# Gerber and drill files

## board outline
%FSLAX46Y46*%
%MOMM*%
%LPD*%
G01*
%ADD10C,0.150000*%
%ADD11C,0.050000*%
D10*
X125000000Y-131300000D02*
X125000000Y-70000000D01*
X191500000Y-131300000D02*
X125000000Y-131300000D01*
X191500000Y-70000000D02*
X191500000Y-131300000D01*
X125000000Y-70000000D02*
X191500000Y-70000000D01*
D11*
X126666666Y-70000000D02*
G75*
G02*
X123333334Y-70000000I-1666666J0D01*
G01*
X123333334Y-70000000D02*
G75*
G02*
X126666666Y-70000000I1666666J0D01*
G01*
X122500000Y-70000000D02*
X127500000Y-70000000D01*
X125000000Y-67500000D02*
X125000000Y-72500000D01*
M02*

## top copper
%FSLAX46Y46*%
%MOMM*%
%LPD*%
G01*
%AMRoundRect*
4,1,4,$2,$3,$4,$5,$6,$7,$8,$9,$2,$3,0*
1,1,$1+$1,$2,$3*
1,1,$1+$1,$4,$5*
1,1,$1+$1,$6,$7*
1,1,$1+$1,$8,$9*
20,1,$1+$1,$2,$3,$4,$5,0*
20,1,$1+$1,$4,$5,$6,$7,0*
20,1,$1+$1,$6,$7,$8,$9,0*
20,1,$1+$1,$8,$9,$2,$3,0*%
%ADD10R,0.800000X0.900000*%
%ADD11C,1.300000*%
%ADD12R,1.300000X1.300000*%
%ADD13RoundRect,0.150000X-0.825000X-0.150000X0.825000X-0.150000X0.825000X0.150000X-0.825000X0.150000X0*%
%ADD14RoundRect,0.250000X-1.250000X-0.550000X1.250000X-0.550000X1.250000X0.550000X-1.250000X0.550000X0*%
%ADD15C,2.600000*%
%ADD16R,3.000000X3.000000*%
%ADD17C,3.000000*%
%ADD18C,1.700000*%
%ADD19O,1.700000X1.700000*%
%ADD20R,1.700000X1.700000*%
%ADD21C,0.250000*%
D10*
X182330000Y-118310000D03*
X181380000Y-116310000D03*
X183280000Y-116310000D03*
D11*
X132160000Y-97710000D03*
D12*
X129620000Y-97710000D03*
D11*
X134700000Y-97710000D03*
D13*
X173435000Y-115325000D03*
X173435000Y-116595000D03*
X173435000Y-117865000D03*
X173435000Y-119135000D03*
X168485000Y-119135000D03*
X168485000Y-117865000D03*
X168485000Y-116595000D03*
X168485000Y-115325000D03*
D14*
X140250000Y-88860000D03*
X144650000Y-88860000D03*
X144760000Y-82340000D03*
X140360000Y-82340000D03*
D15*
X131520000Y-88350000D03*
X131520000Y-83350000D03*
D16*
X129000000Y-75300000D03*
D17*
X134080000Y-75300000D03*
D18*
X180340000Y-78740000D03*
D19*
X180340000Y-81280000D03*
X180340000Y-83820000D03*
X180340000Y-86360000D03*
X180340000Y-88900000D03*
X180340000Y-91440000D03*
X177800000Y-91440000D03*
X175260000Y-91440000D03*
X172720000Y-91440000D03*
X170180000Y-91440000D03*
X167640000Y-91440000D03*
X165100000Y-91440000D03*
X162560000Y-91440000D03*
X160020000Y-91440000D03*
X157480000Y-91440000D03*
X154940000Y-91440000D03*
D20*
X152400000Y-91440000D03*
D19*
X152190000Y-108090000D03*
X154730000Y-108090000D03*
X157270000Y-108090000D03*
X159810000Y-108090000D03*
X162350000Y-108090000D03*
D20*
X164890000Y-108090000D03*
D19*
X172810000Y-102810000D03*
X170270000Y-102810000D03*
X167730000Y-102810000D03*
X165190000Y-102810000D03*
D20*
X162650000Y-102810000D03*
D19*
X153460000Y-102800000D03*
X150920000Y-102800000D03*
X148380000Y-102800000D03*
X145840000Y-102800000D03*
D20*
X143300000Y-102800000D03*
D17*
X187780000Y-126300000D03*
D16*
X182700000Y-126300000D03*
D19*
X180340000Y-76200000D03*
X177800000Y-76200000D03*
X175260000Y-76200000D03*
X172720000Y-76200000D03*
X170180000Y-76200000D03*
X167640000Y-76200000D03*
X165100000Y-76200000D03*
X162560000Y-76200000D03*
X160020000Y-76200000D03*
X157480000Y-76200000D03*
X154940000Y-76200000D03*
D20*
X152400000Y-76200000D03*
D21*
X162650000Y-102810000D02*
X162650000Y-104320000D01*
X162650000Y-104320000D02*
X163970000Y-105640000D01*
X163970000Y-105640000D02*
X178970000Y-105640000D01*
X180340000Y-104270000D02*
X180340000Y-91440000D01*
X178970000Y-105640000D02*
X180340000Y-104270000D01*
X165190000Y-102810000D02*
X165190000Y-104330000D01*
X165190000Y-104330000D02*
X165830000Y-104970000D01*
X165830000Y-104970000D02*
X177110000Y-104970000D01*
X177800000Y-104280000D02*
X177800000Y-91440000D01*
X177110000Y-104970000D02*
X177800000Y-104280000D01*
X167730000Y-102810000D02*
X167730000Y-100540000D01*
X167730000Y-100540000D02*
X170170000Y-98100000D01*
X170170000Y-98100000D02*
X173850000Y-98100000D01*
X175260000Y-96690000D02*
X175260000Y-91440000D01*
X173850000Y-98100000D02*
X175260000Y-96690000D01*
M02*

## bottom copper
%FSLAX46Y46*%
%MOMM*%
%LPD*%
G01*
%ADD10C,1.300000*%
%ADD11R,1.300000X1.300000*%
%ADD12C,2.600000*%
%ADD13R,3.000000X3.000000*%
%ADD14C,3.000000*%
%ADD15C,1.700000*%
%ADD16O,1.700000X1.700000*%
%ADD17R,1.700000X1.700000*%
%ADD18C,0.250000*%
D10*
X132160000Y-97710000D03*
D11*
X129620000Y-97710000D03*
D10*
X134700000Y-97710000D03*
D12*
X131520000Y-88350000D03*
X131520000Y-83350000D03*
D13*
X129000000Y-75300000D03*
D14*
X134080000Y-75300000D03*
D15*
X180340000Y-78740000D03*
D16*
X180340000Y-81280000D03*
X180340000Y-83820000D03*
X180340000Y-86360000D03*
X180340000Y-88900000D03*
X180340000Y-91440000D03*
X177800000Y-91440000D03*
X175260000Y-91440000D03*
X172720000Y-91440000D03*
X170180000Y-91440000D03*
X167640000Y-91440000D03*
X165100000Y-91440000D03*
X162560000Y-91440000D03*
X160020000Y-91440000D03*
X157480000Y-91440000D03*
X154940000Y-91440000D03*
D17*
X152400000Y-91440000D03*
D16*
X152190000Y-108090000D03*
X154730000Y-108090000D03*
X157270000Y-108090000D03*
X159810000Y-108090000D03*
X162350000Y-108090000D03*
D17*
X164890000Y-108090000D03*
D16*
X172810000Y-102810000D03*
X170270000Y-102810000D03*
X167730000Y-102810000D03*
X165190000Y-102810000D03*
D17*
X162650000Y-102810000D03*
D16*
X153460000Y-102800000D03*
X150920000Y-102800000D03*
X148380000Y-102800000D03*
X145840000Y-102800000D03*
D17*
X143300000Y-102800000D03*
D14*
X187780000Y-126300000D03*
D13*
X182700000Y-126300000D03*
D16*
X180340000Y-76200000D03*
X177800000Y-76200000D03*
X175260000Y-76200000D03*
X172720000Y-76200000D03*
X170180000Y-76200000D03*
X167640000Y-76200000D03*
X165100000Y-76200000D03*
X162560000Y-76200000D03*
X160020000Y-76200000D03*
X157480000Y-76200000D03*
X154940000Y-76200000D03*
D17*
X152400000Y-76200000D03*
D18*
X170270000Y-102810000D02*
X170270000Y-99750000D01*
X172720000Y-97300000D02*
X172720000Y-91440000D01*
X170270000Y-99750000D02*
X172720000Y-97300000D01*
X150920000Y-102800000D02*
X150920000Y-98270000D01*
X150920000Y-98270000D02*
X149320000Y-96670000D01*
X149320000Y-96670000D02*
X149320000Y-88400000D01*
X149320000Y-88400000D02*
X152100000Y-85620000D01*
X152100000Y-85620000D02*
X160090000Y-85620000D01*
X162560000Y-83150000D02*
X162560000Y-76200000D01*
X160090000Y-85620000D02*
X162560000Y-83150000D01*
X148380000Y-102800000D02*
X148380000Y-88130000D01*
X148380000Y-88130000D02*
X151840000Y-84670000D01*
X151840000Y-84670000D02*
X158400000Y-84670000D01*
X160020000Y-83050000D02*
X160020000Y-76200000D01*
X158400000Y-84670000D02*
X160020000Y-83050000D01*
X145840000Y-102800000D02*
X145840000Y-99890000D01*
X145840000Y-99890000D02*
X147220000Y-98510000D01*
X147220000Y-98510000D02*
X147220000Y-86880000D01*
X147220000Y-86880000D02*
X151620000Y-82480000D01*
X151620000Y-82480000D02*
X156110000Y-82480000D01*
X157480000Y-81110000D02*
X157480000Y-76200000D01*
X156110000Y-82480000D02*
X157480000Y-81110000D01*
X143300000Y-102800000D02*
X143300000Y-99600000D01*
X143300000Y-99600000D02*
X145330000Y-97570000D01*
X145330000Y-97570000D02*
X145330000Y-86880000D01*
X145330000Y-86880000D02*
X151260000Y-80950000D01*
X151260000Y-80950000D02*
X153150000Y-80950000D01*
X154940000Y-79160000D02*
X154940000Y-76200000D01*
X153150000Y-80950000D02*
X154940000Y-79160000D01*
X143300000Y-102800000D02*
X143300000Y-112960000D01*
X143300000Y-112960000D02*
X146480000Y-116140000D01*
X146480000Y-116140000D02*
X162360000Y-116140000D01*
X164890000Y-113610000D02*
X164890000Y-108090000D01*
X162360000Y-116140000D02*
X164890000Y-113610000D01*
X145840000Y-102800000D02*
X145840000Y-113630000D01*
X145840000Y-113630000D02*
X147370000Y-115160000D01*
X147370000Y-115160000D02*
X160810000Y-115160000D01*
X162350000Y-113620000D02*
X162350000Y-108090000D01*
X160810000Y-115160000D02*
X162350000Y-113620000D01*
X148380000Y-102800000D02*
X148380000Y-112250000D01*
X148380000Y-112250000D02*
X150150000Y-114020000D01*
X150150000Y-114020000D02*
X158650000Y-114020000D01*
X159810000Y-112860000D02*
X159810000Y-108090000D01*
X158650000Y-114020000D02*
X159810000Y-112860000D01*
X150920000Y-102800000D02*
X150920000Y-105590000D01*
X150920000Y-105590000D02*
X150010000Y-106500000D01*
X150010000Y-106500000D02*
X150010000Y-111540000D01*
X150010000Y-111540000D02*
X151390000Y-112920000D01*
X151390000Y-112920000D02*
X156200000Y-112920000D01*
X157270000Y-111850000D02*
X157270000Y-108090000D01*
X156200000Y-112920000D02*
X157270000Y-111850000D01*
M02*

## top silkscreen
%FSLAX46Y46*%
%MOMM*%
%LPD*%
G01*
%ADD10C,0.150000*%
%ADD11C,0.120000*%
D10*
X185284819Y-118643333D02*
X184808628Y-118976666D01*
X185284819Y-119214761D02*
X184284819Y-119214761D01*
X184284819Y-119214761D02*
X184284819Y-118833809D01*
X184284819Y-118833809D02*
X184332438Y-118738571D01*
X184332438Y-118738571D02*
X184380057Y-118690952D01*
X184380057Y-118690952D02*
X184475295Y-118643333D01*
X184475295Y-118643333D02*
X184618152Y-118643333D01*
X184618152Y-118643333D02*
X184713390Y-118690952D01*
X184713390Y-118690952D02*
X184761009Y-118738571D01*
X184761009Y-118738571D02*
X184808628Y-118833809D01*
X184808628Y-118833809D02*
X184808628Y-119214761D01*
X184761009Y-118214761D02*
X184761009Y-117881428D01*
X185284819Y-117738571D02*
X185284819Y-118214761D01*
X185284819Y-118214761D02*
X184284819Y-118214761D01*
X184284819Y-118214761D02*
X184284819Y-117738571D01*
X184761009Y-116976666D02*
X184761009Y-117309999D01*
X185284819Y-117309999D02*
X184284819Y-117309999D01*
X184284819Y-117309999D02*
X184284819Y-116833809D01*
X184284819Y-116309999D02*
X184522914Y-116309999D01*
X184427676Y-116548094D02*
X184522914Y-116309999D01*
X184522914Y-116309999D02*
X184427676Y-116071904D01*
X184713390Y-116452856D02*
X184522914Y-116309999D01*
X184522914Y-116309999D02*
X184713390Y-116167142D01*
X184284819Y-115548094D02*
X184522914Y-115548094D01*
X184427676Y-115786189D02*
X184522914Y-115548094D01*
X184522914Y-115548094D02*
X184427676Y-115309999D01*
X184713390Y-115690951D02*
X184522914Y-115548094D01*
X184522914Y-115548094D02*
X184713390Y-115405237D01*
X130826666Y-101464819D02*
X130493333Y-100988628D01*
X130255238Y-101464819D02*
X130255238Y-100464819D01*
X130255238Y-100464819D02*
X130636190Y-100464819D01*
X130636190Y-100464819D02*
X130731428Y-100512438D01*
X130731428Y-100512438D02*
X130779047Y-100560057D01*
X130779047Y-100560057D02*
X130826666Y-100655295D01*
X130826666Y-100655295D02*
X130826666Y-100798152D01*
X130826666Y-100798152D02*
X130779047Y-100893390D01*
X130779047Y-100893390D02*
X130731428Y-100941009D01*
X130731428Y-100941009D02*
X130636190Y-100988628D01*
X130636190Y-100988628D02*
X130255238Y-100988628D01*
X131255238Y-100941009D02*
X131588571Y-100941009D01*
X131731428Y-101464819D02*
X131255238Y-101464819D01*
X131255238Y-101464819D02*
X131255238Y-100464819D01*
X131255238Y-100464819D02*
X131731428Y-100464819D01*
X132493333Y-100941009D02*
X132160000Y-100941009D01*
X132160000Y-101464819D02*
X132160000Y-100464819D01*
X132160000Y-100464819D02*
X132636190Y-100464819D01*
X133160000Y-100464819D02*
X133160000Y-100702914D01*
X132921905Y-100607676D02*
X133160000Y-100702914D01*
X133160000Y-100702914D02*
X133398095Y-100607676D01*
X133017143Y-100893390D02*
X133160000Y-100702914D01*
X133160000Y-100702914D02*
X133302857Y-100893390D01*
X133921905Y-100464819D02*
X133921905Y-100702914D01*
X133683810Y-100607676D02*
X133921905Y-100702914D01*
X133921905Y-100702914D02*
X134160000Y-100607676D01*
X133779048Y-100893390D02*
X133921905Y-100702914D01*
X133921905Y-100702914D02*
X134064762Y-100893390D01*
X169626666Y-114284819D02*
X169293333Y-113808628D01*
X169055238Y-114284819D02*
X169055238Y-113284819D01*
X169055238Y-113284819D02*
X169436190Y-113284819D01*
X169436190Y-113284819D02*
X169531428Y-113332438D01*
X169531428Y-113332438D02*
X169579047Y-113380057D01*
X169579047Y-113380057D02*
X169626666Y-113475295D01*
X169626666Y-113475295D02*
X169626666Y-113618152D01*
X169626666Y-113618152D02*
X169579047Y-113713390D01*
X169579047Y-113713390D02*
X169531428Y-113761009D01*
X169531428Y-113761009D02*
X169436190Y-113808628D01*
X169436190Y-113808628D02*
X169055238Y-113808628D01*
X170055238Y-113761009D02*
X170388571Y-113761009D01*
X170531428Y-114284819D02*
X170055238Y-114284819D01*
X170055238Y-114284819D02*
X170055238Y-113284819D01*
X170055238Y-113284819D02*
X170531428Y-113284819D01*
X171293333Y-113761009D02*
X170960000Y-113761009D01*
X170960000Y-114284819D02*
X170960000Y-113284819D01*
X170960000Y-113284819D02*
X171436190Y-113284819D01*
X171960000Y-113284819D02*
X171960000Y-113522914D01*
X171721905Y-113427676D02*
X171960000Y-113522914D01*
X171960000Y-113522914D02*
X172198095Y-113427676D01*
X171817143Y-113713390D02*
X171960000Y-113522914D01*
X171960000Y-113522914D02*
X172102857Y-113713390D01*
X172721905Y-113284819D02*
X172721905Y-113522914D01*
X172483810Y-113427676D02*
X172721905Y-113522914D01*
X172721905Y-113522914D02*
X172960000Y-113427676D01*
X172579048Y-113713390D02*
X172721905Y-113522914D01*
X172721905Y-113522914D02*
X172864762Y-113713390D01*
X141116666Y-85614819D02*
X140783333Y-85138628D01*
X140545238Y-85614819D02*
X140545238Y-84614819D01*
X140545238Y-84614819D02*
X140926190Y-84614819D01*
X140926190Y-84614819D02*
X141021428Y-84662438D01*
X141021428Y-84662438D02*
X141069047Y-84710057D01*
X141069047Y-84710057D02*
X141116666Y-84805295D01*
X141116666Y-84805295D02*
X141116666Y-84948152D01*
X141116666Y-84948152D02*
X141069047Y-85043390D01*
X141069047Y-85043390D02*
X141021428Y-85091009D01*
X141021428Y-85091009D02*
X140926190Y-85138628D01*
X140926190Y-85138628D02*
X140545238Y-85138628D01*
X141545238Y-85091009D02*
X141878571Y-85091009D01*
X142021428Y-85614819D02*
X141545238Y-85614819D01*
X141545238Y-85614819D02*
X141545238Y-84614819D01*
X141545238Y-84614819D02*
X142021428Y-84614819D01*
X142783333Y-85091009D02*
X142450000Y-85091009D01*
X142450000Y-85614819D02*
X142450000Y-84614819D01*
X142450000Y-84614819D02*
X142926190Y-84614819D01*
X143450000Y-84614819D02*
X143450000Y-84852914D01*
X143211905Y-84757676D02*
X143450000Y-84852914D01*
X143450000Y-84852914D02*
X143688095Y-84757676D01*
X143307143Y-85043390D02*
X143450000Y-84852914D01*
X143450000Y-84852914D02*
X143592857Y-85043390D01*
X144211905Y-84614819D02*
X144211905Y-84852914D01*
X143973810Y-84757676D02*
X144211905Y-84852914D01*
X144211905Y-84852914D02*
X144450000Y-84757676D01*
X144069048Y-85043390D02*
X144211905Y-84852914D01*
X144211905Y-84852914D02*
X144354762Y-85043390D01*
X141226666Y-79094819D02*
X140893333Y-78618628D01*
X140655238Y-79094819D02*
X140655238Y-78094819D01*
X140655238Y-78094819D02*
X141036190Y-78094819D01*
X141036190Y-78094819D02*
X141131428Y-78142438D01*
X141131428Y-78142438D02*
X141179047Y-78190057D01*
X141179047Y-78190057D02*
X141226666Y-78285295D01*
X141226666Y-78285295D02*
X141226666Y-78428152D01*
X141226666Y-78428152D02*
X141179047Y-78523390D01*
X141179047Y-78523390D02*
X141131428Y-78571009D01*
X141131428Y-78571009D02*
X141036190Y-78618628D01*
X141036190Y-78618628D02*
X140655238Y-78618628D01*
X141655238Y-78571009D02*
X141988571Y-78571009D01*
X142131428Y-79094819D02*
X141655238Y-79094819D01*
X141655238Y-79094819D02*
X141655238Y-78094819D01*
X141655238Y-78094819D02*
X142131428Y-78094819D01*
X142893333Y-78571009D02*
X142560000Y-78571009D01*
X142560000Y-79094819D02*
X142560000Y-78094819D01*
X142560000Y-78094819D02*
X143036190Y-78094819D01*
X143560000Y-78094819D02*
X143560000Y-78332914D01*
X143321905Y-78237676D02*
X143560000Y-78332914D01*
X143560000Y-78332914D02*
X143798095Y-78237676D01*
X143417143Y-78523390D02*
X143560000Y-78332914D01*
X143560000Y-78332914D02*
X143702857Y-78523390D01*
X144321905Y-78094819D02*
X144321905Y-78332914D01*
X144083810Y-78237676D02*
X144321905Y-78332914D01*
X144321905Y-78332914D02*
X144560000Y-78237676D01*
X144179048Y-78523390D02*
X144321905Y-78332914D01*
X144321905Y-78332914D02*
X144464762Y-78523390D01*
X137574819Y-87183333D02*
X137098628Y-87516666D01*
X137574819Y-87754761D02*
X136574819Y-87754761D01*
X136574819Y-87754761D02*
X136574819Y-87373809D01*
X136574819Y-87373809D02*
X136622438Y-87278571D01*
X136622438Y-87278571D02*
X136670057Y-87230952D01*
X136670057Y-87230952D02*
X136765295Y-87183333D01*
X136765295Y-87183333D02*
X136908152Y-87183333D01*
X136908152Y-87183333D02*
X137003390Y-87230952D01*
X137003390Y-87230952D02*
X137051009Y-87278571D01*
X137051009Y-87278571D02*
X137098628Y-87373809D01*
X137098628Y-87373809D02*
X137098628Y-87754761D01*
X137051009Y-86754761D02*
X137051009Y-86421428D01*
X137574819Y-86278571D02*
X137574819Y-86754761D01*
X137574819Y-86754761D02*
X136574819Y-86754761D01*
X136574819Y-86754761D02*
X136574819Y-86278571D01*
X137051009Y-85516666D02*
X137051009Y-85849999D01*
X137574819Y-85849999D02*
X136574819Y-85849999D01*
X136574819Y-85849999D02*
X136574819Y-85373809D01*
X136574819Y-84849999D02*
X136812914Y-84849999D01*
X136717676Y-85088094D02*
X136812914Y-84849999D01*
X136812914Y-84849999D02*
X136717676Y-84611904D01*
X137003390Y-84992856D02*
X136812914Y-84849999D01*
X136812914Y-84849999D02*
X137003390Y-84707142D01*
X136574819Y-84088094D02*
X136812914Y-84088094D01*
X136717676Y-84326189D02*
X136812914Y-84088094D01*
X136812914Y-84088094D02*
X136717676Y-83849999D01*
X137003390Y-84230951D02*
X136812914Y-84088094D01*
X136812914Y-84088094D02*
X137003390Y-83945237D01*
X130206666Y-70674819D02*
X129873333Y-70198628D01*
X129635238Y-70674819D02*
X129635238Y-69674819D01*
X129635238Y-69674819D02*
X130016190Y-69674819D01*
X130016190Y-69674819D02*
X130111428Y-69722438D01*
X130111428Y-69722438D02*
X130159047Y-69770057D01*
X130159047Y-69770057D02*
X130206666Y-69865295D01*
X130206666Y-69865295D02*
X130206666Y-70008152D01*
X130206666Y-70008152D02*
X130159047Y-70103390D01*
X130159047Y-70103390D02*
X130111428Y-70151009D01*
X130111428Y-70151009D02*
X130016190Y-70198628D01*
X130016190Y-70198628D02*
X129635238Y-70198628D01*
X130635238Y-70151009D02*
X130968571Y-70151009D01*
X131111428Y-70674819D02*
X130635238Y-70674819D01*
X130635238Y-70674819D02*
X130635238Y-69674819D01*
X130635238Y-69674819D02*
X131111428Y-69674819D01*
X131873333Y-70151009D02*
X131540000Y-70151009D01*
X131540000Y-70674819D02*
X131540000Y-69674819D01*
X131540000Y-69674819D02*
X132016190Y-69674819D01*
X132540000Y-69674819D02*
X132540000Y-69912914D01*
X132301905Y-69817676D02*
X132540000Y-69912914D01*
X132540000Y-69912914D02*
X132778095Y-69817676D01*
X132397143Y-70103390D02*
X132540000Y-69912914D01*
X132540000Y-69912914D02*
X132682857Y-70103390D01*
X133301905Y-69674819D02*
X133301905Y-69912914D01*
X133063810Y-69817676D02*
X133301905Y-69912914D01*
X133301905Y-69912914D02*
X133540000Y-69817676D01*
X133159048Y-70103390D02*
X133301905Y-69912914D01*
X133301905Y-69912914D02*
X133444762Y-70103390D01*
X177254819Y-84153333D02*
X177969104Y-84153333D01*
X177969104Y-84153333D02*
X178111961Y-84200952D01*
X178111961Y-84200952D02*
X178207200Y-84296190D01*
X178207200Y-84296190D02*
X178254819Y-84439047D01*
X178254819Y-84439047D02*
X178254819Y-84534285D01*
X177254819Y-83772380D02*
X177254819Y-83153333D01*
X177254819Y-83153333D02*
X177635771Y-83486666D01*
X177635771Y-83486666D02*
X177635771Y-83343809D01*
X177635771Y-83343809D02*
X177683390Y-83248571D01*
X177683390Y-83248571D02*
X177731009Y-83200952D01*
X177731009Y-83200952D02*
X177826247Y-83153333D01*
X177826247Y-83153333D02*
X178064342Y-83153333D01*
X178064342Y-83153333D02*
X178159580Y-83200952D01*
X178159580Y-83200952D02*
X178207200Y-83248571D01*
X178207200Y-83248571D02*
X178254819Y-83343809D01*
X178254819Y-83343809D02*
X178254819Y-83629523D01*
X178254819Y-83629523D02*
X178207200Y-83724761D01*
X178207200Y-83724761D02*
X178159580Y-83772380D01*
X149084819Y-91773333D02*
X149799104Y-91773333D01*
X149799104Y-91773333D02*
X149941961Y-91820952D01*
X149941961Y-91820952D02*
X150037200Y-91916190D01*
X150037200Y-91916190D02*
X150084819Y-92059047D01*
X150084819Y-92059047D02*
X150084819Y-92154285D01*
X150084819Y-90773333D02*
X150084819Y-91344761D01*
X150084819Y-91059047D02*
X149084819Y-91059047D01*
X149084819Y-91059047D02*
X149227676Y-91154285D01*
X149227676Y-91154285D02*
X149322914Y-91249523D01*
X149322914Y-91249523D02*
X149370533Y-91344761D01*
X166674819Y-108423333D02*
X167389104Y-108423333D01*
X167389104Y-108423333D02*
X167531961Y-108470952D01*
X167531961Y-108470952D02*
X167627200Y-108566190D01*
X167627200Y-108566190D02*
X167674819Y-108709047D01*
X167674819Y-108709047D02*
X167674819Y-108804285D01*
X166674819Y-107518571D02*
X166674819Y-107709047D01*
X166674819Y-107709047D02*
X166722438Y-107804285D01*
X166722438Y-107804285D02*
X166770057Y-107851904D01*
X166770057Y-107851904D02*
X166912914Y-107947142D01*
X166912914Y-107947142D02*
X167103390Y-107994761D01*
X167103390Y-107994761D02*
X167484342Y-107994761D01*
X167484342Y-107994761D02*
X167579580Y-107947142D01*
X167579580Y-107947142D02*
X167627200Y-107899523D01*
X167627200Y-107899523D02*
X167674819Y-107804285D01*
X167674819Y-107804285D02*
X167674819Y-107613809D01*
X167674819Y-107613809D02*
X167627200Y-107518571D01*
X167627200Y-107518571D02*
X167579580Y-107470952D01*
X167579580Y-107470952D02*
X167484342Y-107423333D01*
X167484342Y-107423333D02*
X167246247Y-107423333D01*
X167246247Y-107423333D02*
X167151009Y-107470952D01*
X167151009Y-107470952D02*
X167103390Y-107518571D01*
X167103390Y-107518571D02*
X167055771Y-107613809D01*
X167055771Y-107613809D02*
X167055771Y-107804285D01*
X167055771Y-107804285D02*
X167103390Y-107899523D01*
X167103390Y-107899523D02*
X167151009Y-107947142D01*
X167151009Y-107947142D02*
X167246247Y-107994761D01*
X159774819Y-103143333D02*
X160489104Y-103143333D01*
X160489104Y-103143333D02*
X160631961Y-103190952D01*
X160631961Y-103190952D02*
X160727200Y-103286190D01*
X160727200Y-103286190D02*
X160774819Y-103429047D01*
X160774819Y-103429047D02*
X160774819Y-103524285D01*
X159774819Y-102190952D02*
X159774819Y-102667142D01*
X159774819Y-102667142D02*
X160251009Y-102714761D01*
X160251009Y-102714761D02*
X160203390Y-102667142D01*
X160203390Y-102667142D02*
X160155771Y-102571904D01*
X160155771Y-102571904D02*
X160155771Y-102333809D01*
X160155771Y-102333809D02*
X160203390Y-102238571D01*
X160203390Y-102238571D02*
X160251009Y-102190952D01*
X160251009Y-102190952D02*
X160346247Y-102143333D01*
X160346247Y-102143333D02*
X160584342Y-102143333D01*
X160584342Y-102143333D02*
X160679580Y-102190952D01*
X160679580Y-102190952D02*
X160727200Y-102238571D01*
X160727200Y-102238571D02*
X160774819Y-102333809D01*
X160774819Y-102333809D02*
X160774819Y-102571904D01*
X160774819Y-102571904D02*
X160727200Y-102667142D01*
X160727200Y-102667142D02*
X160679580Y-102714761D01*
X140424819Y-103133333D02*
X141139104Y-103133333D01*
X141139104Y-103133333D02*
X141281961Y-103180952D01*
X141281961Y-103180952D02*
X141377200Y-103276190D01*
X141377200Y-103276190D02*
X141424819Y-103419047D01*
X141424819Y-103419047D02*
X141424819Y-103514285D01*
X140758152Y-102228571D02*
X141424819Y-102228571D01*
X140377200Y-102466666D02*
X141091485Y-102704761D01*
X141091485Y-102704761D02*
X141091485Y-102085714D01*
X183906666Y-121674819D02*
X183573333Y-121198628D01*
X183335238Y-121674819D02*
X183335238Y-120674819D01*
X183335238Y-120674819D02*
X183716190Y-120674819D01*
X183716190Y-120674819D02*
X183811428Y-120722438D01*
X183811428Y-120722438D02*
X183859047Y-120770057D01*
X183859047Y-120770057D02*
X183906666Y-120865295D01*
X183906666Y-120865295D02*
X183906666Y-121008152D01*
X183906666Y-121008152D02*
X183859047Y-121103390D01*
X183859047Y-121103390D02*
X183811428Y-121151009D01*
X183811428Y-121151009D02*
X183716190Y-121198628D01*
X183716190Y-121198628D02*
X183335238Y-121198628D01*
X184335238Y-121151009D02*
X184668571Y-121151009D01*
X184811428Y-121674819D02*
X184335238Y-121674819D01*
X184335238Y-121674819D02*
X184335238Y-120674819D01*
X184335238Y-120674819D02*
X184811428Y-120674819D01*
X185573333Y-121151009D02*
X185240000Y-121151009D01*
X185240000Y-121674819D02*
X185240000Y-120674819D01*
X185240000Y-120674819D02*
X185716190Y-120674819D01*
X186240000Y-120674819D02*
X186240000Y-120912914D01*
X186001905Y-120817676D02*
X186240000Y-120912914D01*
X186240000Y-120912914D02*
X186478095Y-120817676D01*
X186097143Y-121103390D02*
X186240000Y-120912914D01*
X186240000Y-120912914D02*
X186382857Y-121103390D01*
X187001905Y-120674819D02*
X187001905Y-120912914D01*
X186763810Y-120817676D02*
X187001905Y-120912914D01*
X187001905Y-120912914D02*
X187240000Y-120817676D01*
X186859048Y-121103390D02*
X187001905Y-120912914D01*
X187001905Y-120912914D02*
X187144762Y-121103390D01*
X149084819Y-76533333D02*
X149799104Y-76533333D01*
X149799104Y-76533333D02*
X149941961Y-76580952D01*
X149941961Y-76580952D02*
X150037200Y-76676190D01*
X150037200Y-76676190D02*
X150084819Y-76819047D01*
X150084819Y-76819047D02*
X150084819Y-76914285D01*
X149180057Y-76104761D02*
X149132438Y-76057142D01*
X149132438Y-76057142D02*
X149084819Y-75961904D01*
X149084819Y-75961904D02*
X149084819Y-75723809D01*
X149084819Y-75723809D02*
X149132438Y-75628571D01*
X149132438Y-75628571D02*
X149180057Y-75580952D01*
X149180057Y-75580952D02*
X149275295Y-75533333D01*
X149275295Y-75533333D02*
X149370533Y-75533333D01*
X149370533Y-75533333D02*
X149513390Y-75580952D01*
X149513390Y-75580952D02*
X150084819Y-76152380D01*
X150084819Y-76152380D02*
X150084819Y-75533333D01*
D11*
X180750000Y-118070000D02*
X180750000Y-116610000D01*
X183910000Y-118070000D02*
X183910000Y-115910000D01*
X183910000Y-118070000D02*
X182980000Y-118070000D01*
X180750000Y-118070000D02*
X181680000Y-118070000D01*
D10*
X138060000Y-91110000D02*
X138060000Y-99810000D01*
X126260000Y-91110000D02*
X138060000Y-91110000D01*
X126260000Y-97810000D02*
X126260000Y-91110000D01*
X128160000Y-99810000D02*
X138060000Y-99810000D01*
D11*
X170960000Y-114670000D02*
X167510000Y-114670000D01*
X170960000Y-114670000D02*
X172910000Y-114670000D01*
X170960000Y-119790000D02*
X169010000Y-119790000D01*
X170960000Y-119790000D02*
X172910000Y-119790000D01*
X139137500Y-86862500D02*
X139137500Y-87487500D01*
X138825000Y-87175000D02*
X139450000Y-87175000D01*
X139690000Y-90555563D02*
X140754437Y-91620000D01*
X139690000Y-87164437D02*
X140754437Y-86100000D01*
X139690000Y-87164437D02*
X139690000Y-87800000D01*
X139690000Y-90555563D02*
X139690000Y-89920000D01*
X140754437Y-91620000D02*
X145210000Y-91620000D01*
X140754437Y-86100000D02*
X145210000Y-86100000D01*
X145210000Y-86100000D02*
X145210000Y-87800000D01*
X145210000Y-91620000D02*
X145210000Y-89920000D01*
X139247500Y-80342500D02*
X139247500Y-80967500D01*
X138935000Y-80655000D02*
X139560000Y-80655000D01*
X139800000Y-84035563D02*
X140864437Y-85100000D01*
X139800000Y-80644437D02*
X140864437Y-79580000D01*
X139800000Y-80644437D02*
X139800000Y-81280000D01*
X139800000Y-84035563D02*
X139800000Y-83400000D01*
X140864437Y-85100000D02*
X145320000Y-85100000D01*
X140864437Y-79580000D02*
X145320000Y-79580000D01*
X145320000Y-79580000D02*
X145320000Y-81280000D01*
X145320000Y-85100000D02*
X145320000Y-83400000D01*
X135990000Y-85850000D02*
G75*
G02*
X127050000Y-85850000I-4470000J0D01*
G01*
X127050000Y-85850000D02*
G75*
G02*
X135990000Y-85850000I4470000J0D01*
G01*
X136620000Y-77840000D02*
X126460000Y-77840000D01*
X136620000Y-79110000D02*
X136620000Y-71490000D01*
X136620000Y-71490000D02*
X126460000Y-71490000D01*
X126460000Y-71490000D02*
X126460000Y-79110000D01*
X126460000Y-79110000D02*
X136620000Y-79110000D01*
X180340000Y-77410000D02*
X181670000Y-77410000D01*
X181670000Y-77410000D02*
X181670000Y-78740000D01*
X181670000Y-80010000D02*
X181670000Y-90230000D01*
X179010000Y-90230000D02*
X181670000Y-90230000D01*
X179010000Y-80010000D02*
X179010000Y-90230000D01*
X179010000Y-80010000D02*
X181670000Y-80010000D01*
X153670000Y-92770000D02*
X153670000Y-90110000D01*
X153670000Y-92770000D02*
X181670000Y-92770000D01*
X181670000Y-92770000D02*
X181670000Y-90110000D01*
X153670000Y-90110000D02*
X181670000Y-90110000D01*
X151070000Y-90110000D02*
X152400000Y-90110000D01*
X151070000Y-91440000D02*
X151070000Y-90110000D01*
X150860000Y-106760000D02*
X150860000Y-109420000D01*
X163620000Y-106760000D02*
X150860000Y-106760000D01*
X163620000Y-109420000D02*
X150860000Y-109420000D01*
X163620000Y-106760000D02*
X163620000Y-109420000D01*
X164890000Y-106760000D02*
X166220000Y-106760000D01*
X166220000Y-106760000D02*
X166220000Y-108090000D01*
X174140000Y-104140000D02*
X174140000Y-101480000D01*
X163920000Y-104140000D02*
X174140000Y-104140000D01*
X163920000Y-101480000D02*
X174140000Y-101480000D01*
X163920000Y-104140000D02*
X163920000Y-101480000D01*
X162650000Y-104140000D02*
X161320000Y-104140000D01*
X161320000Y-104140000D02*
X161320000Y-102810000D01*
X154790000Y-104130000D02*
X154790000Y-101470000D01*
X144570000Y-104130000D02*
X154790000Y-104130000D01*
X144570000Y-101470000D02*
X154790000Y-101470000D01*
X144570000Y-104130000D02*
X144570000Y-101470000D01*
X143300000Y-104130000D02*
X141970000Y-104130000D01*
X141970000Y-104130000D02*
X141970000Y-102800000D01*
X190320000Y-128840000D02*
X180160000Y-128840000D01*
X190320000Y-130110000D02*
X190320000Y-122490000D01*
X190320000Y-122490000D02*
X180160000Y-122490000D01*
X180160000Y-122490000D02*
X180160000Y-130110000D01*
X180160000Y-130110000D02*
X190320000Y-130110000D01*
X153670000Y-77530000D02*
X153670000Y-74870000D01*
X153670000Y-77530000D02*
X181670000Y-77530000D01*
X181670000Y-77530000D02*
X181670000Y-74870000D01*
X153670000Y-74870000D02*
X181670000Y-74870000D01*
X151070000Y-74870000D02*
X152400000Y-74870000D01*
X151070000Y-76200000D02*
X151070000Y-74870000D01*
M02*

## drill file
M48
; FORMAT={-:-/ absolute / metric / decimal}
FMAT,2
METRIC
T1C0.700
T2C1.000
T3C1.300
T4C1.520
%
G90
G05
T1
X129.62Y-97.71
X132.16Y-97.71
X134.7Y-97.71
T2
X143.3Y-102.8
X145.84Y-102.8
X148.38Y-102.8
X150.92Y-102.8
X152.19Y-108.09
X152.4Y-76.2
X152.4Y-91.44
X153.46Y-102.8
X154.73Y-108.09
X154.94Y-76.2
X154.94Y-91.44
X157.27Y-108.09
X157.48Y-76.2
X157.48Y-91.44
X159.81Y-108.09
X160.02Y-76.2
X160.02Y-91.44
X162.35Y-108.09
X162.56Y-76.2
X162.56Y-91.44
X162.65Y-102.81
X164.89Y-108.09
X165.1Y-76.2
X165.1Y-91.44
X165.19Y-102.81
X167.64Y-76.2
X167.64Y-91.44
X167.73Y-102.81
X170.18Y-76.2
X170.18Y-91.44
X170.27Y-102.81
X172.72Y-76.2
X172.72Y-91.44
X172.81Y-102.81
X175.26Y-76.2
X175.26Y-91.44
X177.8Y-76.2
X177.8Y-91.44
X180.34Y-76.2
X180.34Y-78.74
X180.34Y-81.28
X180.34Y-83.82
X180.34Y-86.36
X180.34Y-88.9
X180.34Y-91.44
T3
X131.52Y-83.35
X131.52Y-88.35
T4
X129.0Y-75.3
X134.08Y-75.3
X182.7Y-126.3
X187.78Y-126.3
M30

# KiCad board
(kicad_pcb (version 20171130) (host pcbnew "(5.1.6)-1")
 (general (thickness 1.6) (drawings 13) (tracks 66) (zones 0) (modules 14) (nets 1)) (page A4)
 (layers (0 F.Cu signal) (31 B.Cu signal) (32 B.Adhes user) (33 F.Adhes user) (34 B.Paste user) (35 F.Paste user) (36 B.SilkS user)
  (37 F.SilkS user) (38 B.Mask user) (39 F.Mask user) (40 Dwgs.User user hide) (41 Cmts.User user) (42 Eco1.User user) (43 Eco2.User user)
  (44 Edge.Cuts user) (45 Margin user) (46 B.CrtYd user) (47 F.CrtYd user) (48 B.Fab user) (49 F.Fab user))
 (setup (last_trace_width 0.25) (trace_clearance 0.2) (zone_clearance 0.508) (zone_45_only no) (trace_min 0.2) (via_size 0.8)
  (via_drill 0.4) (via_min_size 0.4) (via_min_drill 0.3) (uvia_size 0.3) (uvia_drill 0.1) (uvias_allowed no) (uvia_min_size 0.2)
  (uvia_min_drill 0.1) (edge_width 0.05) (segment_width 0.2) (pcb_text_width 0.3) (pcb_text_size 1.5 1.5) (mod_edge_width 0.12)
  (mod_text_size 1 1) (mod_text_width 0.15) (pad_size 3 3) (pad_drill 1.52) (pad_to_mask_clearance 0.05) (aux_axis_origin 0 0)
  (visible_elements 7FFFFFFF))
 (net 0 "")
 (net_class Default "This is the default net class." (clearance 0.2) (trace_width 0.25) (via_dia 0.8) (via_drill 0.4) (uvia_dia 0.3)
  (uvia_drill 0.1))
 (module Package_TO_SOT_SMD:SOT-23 (layer F.Cu) (at 182.33 117.31 270)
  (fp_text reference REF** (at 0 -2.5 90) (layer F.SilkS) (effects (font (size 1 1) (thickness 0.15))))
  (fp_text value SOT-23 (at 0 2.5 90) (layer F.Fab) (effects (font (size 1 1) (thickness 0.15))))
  (fp_line (start 0.76 1.58) (end -0.7 1.58) (layer F.SilkS) (width 0.12))
  (fp_line (start 0.76 -1.58) (end -1.4 -1.58) (layer F.SilkS) (width 0.12))
  (fp_line (start 0.76 -1.58) (end 0.76 -0.65) (layer F.SilkS) (width 0.12))
  (fp_line (start 0.76 1.58) (end 0.76 0.65) (layer F.SilkS) (width 0.12))
  (pad 3 smd rect (at 1 0 270) (size 0.9 0.8) (layers F.Cu F.Paste F.Mask))
  (pad 2 smd rect (at -1 0.95 270) (size 0.9 0.8) (layers F.Cu F.Paste F.Mask))
  (pad 1 smd rect (at -1 -0.95 270) (size 0.9 0.8) (layers F.Cu F.Paste F.Mask)))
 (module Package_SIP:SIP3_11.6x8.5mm (layer F.Cu) (at 129.62 97.71)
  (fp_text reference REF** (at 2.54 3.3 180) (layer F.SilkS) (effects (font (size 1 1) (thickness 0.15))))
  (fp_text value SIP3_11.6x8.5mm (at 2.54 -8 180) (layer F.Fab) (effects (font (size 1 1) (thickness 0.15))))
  (fp_line (start 8.44 -6.6) (end 8.44 2.1) (layer F.SilkS) (width 0.15))
  (fp_line (start -3.36 -6.6) (end 8.44 -6.6) (layer F.SilkS) (width 0.15))
  (fp_line (start -3.36 0.1) (end -3.36 -6.6) (layer F.SilkS) (width 0.15))
  (fp_line (start -1.46 2.1) (end 8.44 2.1) (layer F.SilkS) (width 0.15))
  (pad 2 thru_hole circle (at 2.54 0 180) (size 1.3 1.3) (drill 0.7) (layers *.Cu *.Mask))
  (pad 1 thru_hole rect (at 0 0 270) (size 1.3 1.3) (drill 0.7) (layers *.Cu *.Mask))
  (pad 3 thru_hole circle (at 5.08 0 270) (size 1.3 1.3) (drill 0.7) (layers *.Cu *.Mask)))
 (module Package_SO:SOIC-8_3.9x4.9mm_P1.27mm (layer F.Cu) (at 170.96 117.23)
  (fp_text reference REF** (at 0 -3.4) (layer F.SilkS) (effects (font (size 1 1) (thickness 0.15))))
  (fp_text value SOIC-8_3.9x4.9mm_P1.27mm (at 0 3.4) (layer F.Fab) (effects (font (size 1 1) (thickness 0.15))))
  (fp_line (start 0 -2.56) (end -3.45 -2.56) (layer F.SilkS) (width 0.12))
  (fp_line (start 0 -2.56) (end 1.95 -2.56) (layer F.SilkS) (width 0.12))
  (fp_line (start 0 2.56) (end -1.95 2.56) (layer F.SilkS) (width 0.12))
  (fp_line (start 0 2.56) (end 1.95 2.56) (layer F.SilkS) (width 0.12))
  (pad 8 smd roundrect (at 2.475 -1.905) (size 1.95 0.6) (layers F.Cu F.Paste F.Mask) (roundrect_rratio 0.25))
  (pad 7 smd roundrect (at 2.475 -0.635) (size 1.95 0.6) (layers F.Cu F.Paste F.Mask) (roundrect_rratio 0.25))
  (pad 6 smd roundrect (at 2.475 0.635) (size 1.95 0.6) (layers F.Cu F.Paste F.Mask) (roundrect_rratio 0.25))
  (pad 5 smd roundrect (at 2.475 1.905) (size 1.95 0.6) (layers F.Cu F.Paste F.Mask) (roundrect_rratio 0.25))
  (pad 4 smd roundrect (at -2.475 1.905) (size 1.95 0.6) (layers F.Cu F.Paste F.Mask) (roundrect_rratio 0.25))
  (pad 3 smd roundrect (at -2.475 0.635) (size 1.95 0.6) (layers F.Cu F.Paste F.Mask) (roundrect_rratio 0.25))
  (pad 2 smd roundrect (at -2.475 -0.635) (size 1.95 0.6) (layers F.Cu F.Paste F.Mask) (roundrect_rratio 0.25))
  (pad 1 smd roundrect (at -2.475 -1.905) (size 1.95 0.6) (layers F.Cu F.Paste F.Mask) (roundrect_rratio 0.25)))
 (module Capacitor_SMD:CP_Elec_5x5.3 (layer F.Cu) (at 142.45 88.86)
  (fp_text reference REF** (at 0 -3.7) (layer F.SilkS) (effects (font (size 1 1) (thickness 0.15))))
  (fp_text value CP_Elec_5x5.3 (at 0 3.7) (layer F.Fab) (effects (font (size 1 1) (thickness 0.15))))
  (fp_line (start -3.3125 -1.9975) (end -3.3125 -1.3725) (layer F.SilkS) (width 0.12))
  (fp_line (start -3.625 -1.685) (end -3 -1.685) (layer F.SilkS) (width 0.12))
  (fp_line (start -2.76 1.695563) (end -1.695563 2.76) (layer F.SilkS) (width 0.12))
  (fp_line (start -2.76 -1.695563) (end -1.695563 -2.76) (layer F.SilkS) (width 0.12))
  (fp_line (start -2.76 -1.695563) (end -2.76 -1.06) (layer F.SilkS) (width 0.12))
  (fp_line (start -2.76 1.695563) (end -2.76 1.06) (layer F.SilkS) (width 0.12))
  (fp_line (start -1.695563 2.76) (end 2.76 2.76) (layer F.SilkS) (width 0.12))
  (fp_line (start -1.695563 -2.76) (end 2.76 -2.76) (layer F.SilkS) (width 0.12))
  (fp_line (start 2.76 -2.76) (end 2.76 -1.06) (layer F.SilkS) (width 0.12))
  (fp_line (start 2.76 2.76) (end 2.76 1.06) (layer F.SilkS) (width 0.12))
  (pad 1 smd roundrect (at -2.2 0) (size 3 1.6) (layers F.Cu F.Paste F.Mask) (roundrect_rratio 0.15625))
  (pad 2 smd roundrect (at 2.2 0) (size 3 1.6) (layers F.Cu F.Paste F.Mask) (roundrect_rratio 0.15625)))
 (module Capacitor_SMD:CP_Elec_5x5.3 (layer F.Cu) (at 142.56 82.34)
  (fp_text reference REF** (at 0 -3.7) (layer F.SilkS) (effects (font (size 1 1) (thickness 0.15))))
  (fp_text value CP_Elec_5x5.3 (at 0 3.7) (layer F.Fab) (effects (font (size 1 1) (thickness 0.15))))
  (fp_line (start -3.3125 -1.9975) (end -3.3125 -1.3725) (layer F.SilkS) (width 0.12))
  (fp_line (start -3.625 -1.685) (end -3 -1.685) (layer F.SilkS) (width 0.12))
  (fp_line (start -2.76 1.695563) (end -1.695563 2.76) (layer F.SilkS) (width 0.12))
  (fp_line (start -2.76 -1.695563) (end -1.695563 -2.76) (layer F.SilkS) (width 0.12))
  (fp_line (start -2.76 -1.695563) (end -2.76 -1.06) (layer F.SilkS) (width 0.12))
  (fp_line (start -2.76 1.695563) (end -2.76 1.06) (layer F.SilkS) (width 0.12))
  (fp_line (start -1.695563 2.76) (end 2.76 2.76) (layer F.SilkS) (width 0.12))
  (fp_line (start -1.695563 -2.76) (end 2.76 -2.76) (layer F.SilkS) (width 0.12))
  (fp_line (start 2.76 -2.76) (end 2.76 -1.06) (layer F.SilkS) (width 0.12))
  (fp_line (start 2.76 2.76) (end 2.76 1.06) (layer F.SilkS) (width 0.12))
  (pad 2 smd roundrect (at 2.2 0) (size 3 1.6) (layers F.Cu F.Paste F.Mask) (roundrect_rratio 0.15625))
  (pad 1 smd roundrect (at -2.2 0) (size 3 1.6) (layers F.Cu F.Paste F.Mask) (roundrect_rratio 0.15625)))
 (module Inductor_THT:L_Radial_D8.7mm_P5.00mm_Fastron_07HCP (layer F.Cu) (at 131.52 83.35 270)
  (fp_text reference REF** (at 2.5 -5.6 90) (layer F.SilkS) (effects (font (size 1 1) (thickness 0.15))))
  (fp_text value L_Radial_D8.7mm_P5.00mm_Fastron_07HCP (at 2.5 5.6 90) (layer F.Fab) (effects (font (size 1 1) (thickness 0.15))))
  (fp_circle (center 2.5 0) (end 6.97 0) (layer F.SilkS) (width 0.12))
  (pad 2 thru_hole circle (at 5 0 270) (size 2.6 2.6) (drill 1.3) (layers *.Cu *.Mask))
  (pad 1 thru_hole circle (at 0 0 270) (size 2.6 2.6) (drill 1.3) (layers *.Cu *.Mask)))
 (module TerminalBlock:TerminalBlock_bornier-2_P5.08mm (layer F.Cu) (at 129 75.3)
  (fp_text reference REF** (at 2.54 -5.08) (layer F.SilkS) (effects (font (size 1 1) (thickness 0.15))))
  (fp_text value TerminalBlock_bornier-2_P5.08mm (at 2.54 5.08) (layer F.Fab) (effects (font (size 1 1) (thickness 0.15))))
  (fp_line (start 7.62 2.54) (end -2.54 2.54) (layer F.SilkS) (width 0.12))
  (fp_line (start 7.62 3.81) (end 7.62 -3.81) (layer F.SilkS) (width 0.12))
  (fp_line (start 7.62 -3.81) (end -2.54 -3.81) (layer F.SilkS) (width 0.12))
  (fp_line (start -2.54 -3.81) (end -2.54 3.81) (layer F.SilkS) (width 0.12))
  (fp_line (start -2.54 3.81) (end 7.62 3.81) (layer F.SilkS) (width 0.12))
  (pad VCC thru_hole rect (at 0 0) (size 3 3) (drill 1.52) (layers *.Cu *.Mask))
  (pad GND thru_hole circle (at 5.08 0) (size 3 3) (drill 1.52) (layers *.Cu *.Mask)))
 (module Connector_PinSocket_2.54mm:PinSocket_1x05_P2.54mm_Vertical (layer F.Cu) (at 180.34 78.74)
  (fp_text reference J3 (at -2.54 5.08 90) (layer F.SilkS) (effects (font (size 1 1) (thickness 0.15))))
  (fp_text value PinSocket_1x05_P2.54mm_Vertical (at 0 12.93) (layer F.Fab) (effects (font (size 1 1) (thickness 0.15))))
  (fp_line (start 0 -1.33) (end 1.33 -1.33) (layer F.SilkS) (width 0.12))
  (fp_line (start 1.33 -1.33) (end 1.33 0) (layer F.SilkS) (width 0.12))
  (fp_line (start 1.33 1.27) (end 1.33 11.49) (layer F.SilkS) (width 0.12))
  (fp_line (start -1.33 11.49) (end 1.33 11.49) (layer F.SilkS) (width 0.12))
  (fp_line (start -1.33 1.27) (end -1.33 11.49) (layer F.SilkS) (width 0.12))
  (fp_line (start -1.33 1.27) (end 1.33 1.27) (layer F.SilkS) (width 0.12))
  (pad TDO thru_hole circle (at 0 0) (size 1.7 1.7) (drill 1) (layers *.Cu *.Mask))
  (pad GND thru_hole oval (at 0 2.54) (size 1.7 1.7) (drill 1) (layers *.Cu *.Mask))
  (pad TDI thru_hole oval (at 0 5.08) (size 1.7 1.7) (drill 1) (layers *.Cu *.Mask))
  (pad TCK thru_hole oval (at 0 7.62) (size 1.7 1.7) (drill 1) (layers *.Cu *.Mask))
  (pad TMS thru_hole oval (at 0 10.16) (size 1.7 1.7) (drill 1) (layers *.Cu *.Mask)))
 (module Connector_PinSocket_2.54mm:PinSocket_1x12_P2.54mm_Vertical (layer F.Cu) (at 152.4 91.44 90)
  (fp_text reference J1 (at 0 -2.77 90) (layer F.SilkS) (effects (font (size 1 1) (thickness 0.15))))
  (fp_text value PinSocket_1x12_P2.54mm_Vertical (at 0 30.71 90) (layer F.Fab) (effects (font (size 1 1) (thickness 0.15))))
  (fp_line (start -1.33 1.27) (end 1.33 1.27) (layer F.SilkS) (width 0.12))
  (fp_line (start -1.33 1.27) (end -1.33 29.27) (layer F.SilkS) (width 0.12))
  (fp_line (start -1.33 29.27) (end 1.33 29.27) (layer F.SilkS) (width 0.12))
  (fp_line (start 1.33 1.27) (end 1.33 29.27) (layer F.SilkS) (width 0.12))
  (fp_line (start 1.33 -1.33) (end 1.33 0) (layer F.SilkS) (width 0.12))
  (fp_line (start 0 -1.33) (end 1.33 -1.33) (layer F.SilkS) (width 0.12))
  (pad taster0 thru_hole oval (at 0 27.94 90) (size 1.7 1.7) (drill 1) (layers *.Cu *.Mask))
  (pad taster1 thru_hole oval (at 0 25.4 90) (size 1.7 1.7) (drill 1) (layers *.Cu *.Mask))
  (pad taster2 thru_hole oval (at 0 22.86 90) (size 1.7 1.7) (drill 1) (layers *.Cu *.Mask))
  (pad taster3 thru_hole oval (at 0 20.32 90) (size 1.7 1.7) (drill 1) (layers *.Cu *.Mask))
  (pad 8 thru_hole oval (at 0 17.78 90) (size 1.7 1.7) (drill 1) (layers *.Cu *.Mask))
  (pad 7 thru_hole oval (at 0 15.24 90) (size 1.7 1.7) (drill 1) (layers *.Cu *.Mask))
  (pad 6 thru_hole oval (at 0 12.7 90) (size 1.7 1.7) (drill 1) (layers *.Cu *.Mask))
  (pad 5 thru_hole oval (at 0 10.16 90) (size 1.7 1.7) (drill 1) (layers *.Cu *.Mask))
  (pad 4 thru_hole oval (at 0 7.62 90) (size 1.7 1.7) (drill 1) (layers *.Cu *.Mask))
  (pad reset thru_hole oval (at 0 5.08 90) (size 1.7 1.7) (drill 1) (layers *.Cu *.Mask))
  (pad 2 thru_hole oval (at 0 2.54 90) (size 1.7 1.7) (drill 1) (layers *.Cu *.Mask))
  (pad GND thru_hole rect (at 0 0 90) (size 1.7 1.7) (drill 1) (layers *.Cu *.Mask)))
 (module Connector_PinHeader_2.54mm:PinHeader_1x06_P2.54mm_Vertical (layer F.Cu) (at 164.89 108.09 270)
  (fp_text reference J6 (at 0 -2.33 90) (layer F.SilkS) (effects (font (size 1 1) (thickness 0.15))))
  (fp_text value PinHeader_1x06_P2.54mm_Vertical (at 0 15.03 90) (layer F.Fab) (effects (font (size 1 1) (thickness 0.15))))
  (fp_line (start -1.33 14.03) (end 1.33 14.03) (layer F.SilkS) (width 0.12))
  (fp_line (start -1.33 1.27) (end -1.33 14.03) (layer F.SilkS) (width 0.12))
  (fp_line (start 1.33 1.27) (end 1.33 14.03) (layer F.SilkS) (width 0.12))
  (fp_line (start -1.33 1.27) (end 1.33 1.27) (layer F.SilkS) (width 0.12))
  (fp_line (start -1.33 0) (end -1.33 -1.33) (layer F.SilkS) (width 0.12))
  (fp_line (start -1.33 -1.33) (end 0 -1.33) (layer F.SilkS) (width 0.12))
  (pad GND thru_hole oval (at 0 12.7 270) (size 1.7 1.7) (drill 1) (layers *.Cu *.Mask))
  (pad VCC thru_hole oval (at 0 10.16 270) (size 1.7 1.7) (drill 1) (layers *.Cu *.Mask))
  (pad ausgang3 thru_hole oval (at 0 7.62 270) (size 1.7 1.7) (drill 1) (layers *.Cu *.Mask))
  (pad ausgang2 thru_hole oval (at 0 5.08 270) (size 1.7 1.7) (drill 1) (layers *.Cu *.Mask))
  (pad ausgang1 thru_hole oval (at 0 2.54 270) (size 1.7 1.7) (drill 1) (layers *.Cu *.Mask))
  (pad ausgang0 thru_hole rect (at 0 0 270) (size 1.7 1.7) (drill 1) (layers *.Cu *.Mask)))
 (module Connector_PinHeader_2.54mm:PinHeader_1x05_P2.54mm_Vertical (layer F.Cu) (at 162.65 102.81 90)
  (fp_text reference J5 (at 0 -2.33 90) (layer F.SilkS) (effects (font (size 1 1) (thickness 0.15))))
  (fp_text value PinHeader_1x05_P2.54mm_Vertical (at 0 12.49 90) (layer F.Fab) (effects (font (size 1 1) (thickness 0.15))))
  (fp_line (start -1.33 11.49) (end 1.33 11.49) (layer F.SilkS) (width 0.12))
  (fp_line (start -1.33 1.27) (end -1.33 11.49) (layer F.SilkS) (width 0.12))
  (fp_line (start 1.33 1.27) (end 1.33 11.49) (layer F.SilkS) (width 0.12))
  (fp_line (start -1.33 1.27) (end 1.33 1.27) (layer F.SilkS) (width 0.12))
  (fp_line (start -1.33 0) (end -1.33 -1.33) (layer F.SilkS) (width 0.12))
  (fp_line (start -1.33 -1.33) (end 0 -1.33) (layer F.SilkS) (width 0.12))
  (pad GND thru_hole oval (at 0 10.16 90) (size 1.7 1.7) (drill 1) (layers *.Cu *.Mask))
  (pad taster3 thru_hole oval (at 0 7.62 90) (size 1.7 1.7) (drill 1) (layers *.Cu *.Mask))
  (pad taster2 thru_hole oval (at 0 5.08 90) (size 1.7 1.7) (drill 1) (layers *.Cu *.Mask))
  (pad taster1 thru_hole oval (at 0 2.54 90) (size 1.7 1.7) (drill 1) (layers *.Cu *.Mask))
  (pad taster0 thru_hole rect (at 0 0 90) (size 1.7 1.7) (drill 1) (layers *.Cu *.Mask)))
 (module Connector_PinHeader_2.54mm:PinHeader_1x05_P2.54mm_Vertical (layer F.Cu) (at 143.3 102.8 90)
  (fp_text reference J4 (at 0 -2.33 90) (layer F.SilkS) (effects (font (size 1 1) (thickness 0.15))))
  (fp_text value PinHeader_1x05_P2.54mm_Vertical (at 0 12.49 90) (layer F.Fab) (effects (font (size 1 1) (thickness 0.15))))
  (fp_line (start -1.33 11.49) (end 1.33 11.49) (layer F.SilkS) (width 0.12))
  (fp_line (start -1.33 1.27) (end -1.33 11.49) (layer F.SilkS) (width 0.12))
  (fp_line (start 1.33 1.27) (end 1.33 11.49) (layer F.SilkS) (width 0.12))
  (fp_line (start -1.33 1.27) (end 1.33 1.27) (layer F.SilkS) (width 0.12))
  (fp_line (start -1.33 0) (end -1.33 -1.33) (layer F.SilkS) (width 0.12))
  (fp_line (start -1.33 -1.33) (end 0 -1.33) (layer F.SilkS) (width 0.12))
  (pad GND thru_hole oval (at 0 10.16 90) (size 1.7 1.7) (drill 1) (layers *.Cu *.Mask))
  (pad ausgang3 thru_hole oval (at 0 7.62 90) (size 1.7 1.7) (drill 1) (layers *.Cu *.Mask))
  (pad ausgang2 thru_hole oval (at 0 5.08 90) (size 1.7 1.7) (drill 1) (layers *.Cu *.Mask))
  (pad ausgang1 thru_hole oval (at 0 2.54 90) (size 1.7 1.7) (drill 1) (layers *.Cu *.Mask))
  (pad ausgang0 thru_hole rect (at 0 0 90) (size 1.7 1.7) (drill 1) (layers *.Cu *.Mask)))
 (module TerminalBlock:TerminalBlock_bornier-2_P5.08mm (layer F.Cu) (at 182.7 126.3)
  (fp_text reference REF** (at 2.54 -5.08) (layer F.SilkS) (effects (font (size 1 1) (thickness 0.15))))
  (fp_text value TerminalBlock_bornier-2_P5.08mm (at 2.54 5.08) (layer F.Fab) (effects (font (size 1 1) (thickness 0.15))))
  (fp_line (start 7.62 2.54) (end -2.54 2.54) (layer F.SilkS) (width 0.12))
  (fp_line (start 7.62 3.81) (end 7.62 -3.81) (layer F.SilkS) (width 0.12))
  (fp_line (start 7.62 -3.81) (end -2.54 -3.81) (layer F.SilkS) (width 0.12))
  (fp_line (start -2.54 -3.81) (end -2.54 3.81) (layer F.SilkS) (width 0.12))
  (fp_line (start -2.54 3.81) (end 7.62 3.81) (layer F.SilkS) (width 0.12))
  (pad 2 thru_hole circle (at 5.08 0) (size 3 3) (drill 1.52) (layers *.Cu *.Mask))
  (pad 1 thru_hole rect (at 0 0) (size 3 3) (drill 1.52) (layers *.Cu *.Mask)))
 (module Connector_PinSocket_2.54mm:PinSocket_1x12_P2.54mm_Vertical (layer F.Cu) (at 152.4 76.2 90)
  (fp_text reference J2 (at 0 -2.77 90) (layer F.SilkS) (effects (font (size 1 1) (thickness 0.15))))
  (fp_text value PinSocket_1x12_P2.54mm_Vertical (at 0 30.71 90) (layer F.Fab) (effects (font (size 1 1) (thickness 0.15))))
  (fp_line (start -1.33 1.27) (end 1.33 1.27) (layer F.SilkS) (width 0.12))
  (fp_line (start -1.33 1.27) (end -1.33 29.27) (layer F.SilkS) (width 0.12))
  (fp_line (start -1.33 29.27) (end 1.33 29.27) (layer F.SilkS) (width 0.12))
  (fp_line (start 1.33 1.27) (end 1.33 29.27) (layer F.SilkS) (width 0.12))
  (fp_line (start 1.33 -1.33) (end 1.33 0) (layer F.SilkS) (width 0.12))
  (fp_line (start 0 -1.33) (end 1.33 -1.33) (layer F.SilkS) (width 0.12))
  (pad 12 thru_hole oval (at 0 27.94 90) (size 1.7 1.7) (drill 1) (layers *.Cu *.Mask))
  (pad 11 thru_hole oval (at 0 25.4 90) (size 1.7 1.7) (drill 1) (layers *.Cu *.Mask))
  (pad 10 thru_hole oval (at 0 22.86 90) (size 1.7 1.7) (drill 1) (layers *.Cu *.Mask))
  (pad 9 thru_hole oval (at 0 20.32 90) (size 1.7 1.7) (drill 1) (layers *.Cu *.Mask))
  (pad in_serial thru_hole oval (at 0 17.78 90) (size 1.7 1.7) (drill 1) (layers *.Cu *.Mask))
  (pad out_serial thru_hole oval (at 0 15.24 90) (size 1.7 1.7) (drill 1) (layers *.Cu *.Mask))
  (pad serial_enable thru_hole oval (at 0 12.7 90) (size 1.7 1.7) (drill 1) (layers *.Cu *.Mask))
  (pad ausgang3 thru_hole oval (at 0 10.16 90) (size 1.7 1.7) (drill 1) (layers *.Cu *.Mask))
  (pad ausgang2 thru_hole oval (at 0 7.62 90) (size 1.7 1.7) (drill 1) (layers *.Cu *.Mask))
  (pad ausgang1 thru_hole oval (at 0 5.08 90) (size 1.7 1.7) (drill 1) (layers *.Cu *.Mask))
  (pad ausgang0 thru_hole oval (at 0 2.54 90) (size 1.7 1.7) (drill 1) (layers *.Cu *.Mask))
  (pad 3.3v thru_hole rect (at 0 0 90) (size 1.7 1.7) (drill 1) (layers *.Cu *.Mask)))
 (gr_line (start 125 131.3) (end 125 70) (layer Edge.Cuts) (width 0.15))
 (gr_line (start 191.5 131.3) (end 125 131.3) (layer Edge.Cuts) (width 0.15))
 (gr_line (start 191.5 70) (end 191.5 131.3) (layer Edge.Cuts) (width 0.15))
 (gr_line (start 125 70) (end 191.5 70) (layer Edge.Cuts) (width 0.15))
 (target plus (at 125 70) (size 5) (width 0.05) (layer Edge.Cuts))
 (segment (start 162.65 102.81) (end 162.65 104.32) (width 0.25) (layer F.Cu) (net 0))
 (segment (start 162.65 104.32) (end 163.97 105.64) (width 0.25) (layer F.Cu) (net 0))
 (segment (start 163.97 105.64) (end 178.97 105.64) (width 0.25) (layer F.Cu) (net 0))
 (segment (start 180.34 104.27) (end 180.34 91.44) (width 0.25) (layer F.Cu) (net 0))
 (segment (start 178.97 105.64) (end 180.34 104.27) (width 0.25) (layer F.Cu) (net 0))
 (segment (start 165.19 102.81) (end 165.19 104.33) (width 0.25) (layer F.Cu) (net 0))
 (segment (start 165.19 104.33) (end 165.83 104.97) (width 0.25) (layer F.Cu) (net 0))
 (segment (start 165.83 104.97) (end 177.11 104.97) (width 0.25) (layer F.Cu) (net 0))
 (segment (start 177.8 104.28) (end 177.8 91.44) (width 0.25) (layer F.Cu) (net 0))
 (segment (start 177.11 104.97) (end 177.8 104.28) (width 0.25) (layer F.Cu) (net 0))
 (segment (start 167.73 102.81) (end 167.73 100.54) (width 0.25) (layer F.Cu) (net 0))
 (segment (start 167.73 100.54) (end 170.17 98.1) (width 0.25) (layer F.Cu) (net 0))
 (segment (start 170.17 98.1) (end 173.85 98.1) (width 0.25) (layer F.Cu) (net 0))
 (segment (start 175.26 96.69) (end 175.26 91.44) (width 0.25) (layer F.Cu) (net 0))
 (segment (start 173.85 98.1) (end 175.26 96.69) (width 0.25) (layer F.Cu) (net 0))
 (segment (start 170.27 102.81) (end 170.27 99.75) (width 0.25) (layer B.Cu) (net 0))
 (segment (start 172.72 97.3) (end 172.72 91.44) (width 0.25) (layer B.Cu) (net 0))
 (segment (start 170.27 99.75) (end 172.72 97.3) (width 0.25) (layer B.Cu) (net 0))
 (segment (start 150.92 102.8) (end 150.92 98.27) (width 0.25) (layer B.Cu) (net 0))
 (segment (start 150.92 98.27) (end 149.32 96.67) (width 0.25) (layer B.Cu) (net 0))
 (segment (start 149.32 96.67) (end 149.32 88.4) (width 0.25) (layer B.Cu) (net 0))
 (segment (start 149.32 88.4) (end 152.1 85.62) (width 0.25) (layer B.Cu) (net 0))
 (segment (start 152.1 85.62) (end 160.09 85.62) (width 0.25) (layer B.Cu) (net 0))
 (segment (start 162.56 83.15) (end 162.56 76.2) (width 0.25) (layer B.Cu) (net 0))
 (segment (start 160.09 85.62) (end 162.56 83.15) (width 0.25) (layer B.Cu) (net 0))
 (segment (start 148.38 102.8) (end 148.38 88.13) (width 0.25) (layer B.Cu) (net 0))
 (segment (start 148.38 88.13) (end 151.84 84.67) (width 0.25) (layer B.Cu) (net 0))
 (segment (start 151.84 84.67) (end 158.4 84.67) (width 0.25) (layer B.Cu) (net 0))
 (segment (start 160.02 83.05) (end 160.02 76.2) (width 0.25) (layer B.Cu) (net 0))
 (segment (start 158.4 84.67) (end 160.02 83.05) (width 0.25) (layer B.Cu) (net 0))
 (segment (start 145.84 102.8) (end 145.84 99.89) (width 0.25) (layer B.Cu) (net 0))
 (segment (start 145.84 99.89) (end 147.22 98.51) (width 0.25) (layer B.Cu) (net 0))
 (segment (start 147.22 98.51) (end 147.22 86.88) (width 0.25) (layer B.Cu) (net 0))
 (segment (start 147.22 86.88) (end 151.62 82.48) (width 0.25) (layer B.Cu) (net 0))
 (segment (start 151.62 82.48) (end 156.11 82.48) (width 0.25) (layer B.Cu) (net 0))
 (segment (start 157.48 81.11) (end 157.48 76.2) (width 0.25) (layer B.Cu) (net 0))
 (segment (start 156.11 82.48) (end 157.48 81.11) (width 0.25) (layer B.Cu) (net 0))
 (segment (start 143.3 102.8) (end 143.3 99.6) (width 0.25) (layer B.Cu) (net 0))
 (segment (start 143.3 99.6) (end 145.33 97.57) (width 0.25) (layer B.Cu) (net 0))
 (segment (start 145.33 97.57) (end 145.33 86.88) (width 0.25) (layer B.Cu) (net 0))
 (segment (start 145.33 86.88) (end 151.26 80.95) (width 0.25) (layer B.Cu) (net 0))
 (segment (start 151.26 80.95) (end 153.15 80.95) (width 0.25) (layer B.Cu) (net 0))
 (segment (start 154.94 79.16) (end 154.94 76.2) (width 0.25) (layer B.Cu) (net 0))
 (segment (start 153.15 80.95) (end 154.94 79.16) (width 0.25) (layer B.Cu) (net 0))
 (segment (start 143.3 102.8) (end 143.3 112.96) (width 0.25) (layer B.Cu) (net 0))
 (segment (start 143.3 112.96) (end 146.48 116.14) (width 0.25) (layer B.Cu) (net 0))
 (segment (start 146.48 116.14) (end 162.36 116.14) (width 0.25) (layer B.Cu) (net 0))
 (segment (start 164.89 113.61) (end 164.89 108.09) (width 0.25) (layer B.Cu) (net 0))
 (segment (start 162.36 116.14) (end 164.89 113.61) (width 0.25) (layer B.Cu) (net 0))
 (segment (start 145.84 102.8) (end 145.84 113.63) (width 0.25) (layer B.Cu) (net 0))
 (segment (start 145.84 113.63) (end 147.37 115.16) (width 0.25) (layer B.Cu) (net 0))
 (segment (start 147.37 115.16) (end 160.81 115.16) (width 0.25) (layer B.Cu) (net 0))
 (segment (start 162.35 113.62) (end 162.35 108.09) (width 0.25) (layer B.Cu) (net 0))
 (segment (start 160.81 115.16) (end 162.35 113.62) (width 0.25) (layer B.Cu) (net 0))
 (segment (start 148.38 102.8) (end 148.38 112.25) (width 0.25) (layer B.Cu) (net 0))
 (segment (start 148.38 112.25) (end 150.15 114.02) (width 0.25) (layer B.Cu) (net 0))
 (segment (start 150.15 114.02) (end 158.65 114.02) (width 0.25) (layer B.Cu) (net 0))
 (segment (start 159.81 112.86) (end 159.81 108.09) (width 0.25) (layer B.Cu) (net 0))
 (segment (start 158.65 114.02) (end 159.81 112.86) (width 0.25) (layer B.Cu) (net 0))
 (segment (start 150.92 102.8) (end 150.92 105.59) (width 0.25) (layer B.Cu) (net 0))
 (segment (start 150.92 105.59) (end 150.01 106.5) (width 0.25) (layer B.Cu) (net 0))
 (segment (start 150.01 106.5) (end 150.01 111.54) (width 0.25) (layer B.Cu) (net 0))
 (segment (start 150.01 111.54) (end 151.39 112.92) (width 0.25) (layer B.Cu) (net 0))
 (segment (start 151.39 112.92) (end 156.2 112.92) (width 0.25) (layer B.Cu) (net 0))
 (segment (start 157.27 111.85) (end 157.27 108.09) (width 0.25) (layer B.Cu) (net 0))
 (segment (start 156.2 112.92) (end 157.27 111.85) (width 0.25) (layer B.Cu) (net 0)))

